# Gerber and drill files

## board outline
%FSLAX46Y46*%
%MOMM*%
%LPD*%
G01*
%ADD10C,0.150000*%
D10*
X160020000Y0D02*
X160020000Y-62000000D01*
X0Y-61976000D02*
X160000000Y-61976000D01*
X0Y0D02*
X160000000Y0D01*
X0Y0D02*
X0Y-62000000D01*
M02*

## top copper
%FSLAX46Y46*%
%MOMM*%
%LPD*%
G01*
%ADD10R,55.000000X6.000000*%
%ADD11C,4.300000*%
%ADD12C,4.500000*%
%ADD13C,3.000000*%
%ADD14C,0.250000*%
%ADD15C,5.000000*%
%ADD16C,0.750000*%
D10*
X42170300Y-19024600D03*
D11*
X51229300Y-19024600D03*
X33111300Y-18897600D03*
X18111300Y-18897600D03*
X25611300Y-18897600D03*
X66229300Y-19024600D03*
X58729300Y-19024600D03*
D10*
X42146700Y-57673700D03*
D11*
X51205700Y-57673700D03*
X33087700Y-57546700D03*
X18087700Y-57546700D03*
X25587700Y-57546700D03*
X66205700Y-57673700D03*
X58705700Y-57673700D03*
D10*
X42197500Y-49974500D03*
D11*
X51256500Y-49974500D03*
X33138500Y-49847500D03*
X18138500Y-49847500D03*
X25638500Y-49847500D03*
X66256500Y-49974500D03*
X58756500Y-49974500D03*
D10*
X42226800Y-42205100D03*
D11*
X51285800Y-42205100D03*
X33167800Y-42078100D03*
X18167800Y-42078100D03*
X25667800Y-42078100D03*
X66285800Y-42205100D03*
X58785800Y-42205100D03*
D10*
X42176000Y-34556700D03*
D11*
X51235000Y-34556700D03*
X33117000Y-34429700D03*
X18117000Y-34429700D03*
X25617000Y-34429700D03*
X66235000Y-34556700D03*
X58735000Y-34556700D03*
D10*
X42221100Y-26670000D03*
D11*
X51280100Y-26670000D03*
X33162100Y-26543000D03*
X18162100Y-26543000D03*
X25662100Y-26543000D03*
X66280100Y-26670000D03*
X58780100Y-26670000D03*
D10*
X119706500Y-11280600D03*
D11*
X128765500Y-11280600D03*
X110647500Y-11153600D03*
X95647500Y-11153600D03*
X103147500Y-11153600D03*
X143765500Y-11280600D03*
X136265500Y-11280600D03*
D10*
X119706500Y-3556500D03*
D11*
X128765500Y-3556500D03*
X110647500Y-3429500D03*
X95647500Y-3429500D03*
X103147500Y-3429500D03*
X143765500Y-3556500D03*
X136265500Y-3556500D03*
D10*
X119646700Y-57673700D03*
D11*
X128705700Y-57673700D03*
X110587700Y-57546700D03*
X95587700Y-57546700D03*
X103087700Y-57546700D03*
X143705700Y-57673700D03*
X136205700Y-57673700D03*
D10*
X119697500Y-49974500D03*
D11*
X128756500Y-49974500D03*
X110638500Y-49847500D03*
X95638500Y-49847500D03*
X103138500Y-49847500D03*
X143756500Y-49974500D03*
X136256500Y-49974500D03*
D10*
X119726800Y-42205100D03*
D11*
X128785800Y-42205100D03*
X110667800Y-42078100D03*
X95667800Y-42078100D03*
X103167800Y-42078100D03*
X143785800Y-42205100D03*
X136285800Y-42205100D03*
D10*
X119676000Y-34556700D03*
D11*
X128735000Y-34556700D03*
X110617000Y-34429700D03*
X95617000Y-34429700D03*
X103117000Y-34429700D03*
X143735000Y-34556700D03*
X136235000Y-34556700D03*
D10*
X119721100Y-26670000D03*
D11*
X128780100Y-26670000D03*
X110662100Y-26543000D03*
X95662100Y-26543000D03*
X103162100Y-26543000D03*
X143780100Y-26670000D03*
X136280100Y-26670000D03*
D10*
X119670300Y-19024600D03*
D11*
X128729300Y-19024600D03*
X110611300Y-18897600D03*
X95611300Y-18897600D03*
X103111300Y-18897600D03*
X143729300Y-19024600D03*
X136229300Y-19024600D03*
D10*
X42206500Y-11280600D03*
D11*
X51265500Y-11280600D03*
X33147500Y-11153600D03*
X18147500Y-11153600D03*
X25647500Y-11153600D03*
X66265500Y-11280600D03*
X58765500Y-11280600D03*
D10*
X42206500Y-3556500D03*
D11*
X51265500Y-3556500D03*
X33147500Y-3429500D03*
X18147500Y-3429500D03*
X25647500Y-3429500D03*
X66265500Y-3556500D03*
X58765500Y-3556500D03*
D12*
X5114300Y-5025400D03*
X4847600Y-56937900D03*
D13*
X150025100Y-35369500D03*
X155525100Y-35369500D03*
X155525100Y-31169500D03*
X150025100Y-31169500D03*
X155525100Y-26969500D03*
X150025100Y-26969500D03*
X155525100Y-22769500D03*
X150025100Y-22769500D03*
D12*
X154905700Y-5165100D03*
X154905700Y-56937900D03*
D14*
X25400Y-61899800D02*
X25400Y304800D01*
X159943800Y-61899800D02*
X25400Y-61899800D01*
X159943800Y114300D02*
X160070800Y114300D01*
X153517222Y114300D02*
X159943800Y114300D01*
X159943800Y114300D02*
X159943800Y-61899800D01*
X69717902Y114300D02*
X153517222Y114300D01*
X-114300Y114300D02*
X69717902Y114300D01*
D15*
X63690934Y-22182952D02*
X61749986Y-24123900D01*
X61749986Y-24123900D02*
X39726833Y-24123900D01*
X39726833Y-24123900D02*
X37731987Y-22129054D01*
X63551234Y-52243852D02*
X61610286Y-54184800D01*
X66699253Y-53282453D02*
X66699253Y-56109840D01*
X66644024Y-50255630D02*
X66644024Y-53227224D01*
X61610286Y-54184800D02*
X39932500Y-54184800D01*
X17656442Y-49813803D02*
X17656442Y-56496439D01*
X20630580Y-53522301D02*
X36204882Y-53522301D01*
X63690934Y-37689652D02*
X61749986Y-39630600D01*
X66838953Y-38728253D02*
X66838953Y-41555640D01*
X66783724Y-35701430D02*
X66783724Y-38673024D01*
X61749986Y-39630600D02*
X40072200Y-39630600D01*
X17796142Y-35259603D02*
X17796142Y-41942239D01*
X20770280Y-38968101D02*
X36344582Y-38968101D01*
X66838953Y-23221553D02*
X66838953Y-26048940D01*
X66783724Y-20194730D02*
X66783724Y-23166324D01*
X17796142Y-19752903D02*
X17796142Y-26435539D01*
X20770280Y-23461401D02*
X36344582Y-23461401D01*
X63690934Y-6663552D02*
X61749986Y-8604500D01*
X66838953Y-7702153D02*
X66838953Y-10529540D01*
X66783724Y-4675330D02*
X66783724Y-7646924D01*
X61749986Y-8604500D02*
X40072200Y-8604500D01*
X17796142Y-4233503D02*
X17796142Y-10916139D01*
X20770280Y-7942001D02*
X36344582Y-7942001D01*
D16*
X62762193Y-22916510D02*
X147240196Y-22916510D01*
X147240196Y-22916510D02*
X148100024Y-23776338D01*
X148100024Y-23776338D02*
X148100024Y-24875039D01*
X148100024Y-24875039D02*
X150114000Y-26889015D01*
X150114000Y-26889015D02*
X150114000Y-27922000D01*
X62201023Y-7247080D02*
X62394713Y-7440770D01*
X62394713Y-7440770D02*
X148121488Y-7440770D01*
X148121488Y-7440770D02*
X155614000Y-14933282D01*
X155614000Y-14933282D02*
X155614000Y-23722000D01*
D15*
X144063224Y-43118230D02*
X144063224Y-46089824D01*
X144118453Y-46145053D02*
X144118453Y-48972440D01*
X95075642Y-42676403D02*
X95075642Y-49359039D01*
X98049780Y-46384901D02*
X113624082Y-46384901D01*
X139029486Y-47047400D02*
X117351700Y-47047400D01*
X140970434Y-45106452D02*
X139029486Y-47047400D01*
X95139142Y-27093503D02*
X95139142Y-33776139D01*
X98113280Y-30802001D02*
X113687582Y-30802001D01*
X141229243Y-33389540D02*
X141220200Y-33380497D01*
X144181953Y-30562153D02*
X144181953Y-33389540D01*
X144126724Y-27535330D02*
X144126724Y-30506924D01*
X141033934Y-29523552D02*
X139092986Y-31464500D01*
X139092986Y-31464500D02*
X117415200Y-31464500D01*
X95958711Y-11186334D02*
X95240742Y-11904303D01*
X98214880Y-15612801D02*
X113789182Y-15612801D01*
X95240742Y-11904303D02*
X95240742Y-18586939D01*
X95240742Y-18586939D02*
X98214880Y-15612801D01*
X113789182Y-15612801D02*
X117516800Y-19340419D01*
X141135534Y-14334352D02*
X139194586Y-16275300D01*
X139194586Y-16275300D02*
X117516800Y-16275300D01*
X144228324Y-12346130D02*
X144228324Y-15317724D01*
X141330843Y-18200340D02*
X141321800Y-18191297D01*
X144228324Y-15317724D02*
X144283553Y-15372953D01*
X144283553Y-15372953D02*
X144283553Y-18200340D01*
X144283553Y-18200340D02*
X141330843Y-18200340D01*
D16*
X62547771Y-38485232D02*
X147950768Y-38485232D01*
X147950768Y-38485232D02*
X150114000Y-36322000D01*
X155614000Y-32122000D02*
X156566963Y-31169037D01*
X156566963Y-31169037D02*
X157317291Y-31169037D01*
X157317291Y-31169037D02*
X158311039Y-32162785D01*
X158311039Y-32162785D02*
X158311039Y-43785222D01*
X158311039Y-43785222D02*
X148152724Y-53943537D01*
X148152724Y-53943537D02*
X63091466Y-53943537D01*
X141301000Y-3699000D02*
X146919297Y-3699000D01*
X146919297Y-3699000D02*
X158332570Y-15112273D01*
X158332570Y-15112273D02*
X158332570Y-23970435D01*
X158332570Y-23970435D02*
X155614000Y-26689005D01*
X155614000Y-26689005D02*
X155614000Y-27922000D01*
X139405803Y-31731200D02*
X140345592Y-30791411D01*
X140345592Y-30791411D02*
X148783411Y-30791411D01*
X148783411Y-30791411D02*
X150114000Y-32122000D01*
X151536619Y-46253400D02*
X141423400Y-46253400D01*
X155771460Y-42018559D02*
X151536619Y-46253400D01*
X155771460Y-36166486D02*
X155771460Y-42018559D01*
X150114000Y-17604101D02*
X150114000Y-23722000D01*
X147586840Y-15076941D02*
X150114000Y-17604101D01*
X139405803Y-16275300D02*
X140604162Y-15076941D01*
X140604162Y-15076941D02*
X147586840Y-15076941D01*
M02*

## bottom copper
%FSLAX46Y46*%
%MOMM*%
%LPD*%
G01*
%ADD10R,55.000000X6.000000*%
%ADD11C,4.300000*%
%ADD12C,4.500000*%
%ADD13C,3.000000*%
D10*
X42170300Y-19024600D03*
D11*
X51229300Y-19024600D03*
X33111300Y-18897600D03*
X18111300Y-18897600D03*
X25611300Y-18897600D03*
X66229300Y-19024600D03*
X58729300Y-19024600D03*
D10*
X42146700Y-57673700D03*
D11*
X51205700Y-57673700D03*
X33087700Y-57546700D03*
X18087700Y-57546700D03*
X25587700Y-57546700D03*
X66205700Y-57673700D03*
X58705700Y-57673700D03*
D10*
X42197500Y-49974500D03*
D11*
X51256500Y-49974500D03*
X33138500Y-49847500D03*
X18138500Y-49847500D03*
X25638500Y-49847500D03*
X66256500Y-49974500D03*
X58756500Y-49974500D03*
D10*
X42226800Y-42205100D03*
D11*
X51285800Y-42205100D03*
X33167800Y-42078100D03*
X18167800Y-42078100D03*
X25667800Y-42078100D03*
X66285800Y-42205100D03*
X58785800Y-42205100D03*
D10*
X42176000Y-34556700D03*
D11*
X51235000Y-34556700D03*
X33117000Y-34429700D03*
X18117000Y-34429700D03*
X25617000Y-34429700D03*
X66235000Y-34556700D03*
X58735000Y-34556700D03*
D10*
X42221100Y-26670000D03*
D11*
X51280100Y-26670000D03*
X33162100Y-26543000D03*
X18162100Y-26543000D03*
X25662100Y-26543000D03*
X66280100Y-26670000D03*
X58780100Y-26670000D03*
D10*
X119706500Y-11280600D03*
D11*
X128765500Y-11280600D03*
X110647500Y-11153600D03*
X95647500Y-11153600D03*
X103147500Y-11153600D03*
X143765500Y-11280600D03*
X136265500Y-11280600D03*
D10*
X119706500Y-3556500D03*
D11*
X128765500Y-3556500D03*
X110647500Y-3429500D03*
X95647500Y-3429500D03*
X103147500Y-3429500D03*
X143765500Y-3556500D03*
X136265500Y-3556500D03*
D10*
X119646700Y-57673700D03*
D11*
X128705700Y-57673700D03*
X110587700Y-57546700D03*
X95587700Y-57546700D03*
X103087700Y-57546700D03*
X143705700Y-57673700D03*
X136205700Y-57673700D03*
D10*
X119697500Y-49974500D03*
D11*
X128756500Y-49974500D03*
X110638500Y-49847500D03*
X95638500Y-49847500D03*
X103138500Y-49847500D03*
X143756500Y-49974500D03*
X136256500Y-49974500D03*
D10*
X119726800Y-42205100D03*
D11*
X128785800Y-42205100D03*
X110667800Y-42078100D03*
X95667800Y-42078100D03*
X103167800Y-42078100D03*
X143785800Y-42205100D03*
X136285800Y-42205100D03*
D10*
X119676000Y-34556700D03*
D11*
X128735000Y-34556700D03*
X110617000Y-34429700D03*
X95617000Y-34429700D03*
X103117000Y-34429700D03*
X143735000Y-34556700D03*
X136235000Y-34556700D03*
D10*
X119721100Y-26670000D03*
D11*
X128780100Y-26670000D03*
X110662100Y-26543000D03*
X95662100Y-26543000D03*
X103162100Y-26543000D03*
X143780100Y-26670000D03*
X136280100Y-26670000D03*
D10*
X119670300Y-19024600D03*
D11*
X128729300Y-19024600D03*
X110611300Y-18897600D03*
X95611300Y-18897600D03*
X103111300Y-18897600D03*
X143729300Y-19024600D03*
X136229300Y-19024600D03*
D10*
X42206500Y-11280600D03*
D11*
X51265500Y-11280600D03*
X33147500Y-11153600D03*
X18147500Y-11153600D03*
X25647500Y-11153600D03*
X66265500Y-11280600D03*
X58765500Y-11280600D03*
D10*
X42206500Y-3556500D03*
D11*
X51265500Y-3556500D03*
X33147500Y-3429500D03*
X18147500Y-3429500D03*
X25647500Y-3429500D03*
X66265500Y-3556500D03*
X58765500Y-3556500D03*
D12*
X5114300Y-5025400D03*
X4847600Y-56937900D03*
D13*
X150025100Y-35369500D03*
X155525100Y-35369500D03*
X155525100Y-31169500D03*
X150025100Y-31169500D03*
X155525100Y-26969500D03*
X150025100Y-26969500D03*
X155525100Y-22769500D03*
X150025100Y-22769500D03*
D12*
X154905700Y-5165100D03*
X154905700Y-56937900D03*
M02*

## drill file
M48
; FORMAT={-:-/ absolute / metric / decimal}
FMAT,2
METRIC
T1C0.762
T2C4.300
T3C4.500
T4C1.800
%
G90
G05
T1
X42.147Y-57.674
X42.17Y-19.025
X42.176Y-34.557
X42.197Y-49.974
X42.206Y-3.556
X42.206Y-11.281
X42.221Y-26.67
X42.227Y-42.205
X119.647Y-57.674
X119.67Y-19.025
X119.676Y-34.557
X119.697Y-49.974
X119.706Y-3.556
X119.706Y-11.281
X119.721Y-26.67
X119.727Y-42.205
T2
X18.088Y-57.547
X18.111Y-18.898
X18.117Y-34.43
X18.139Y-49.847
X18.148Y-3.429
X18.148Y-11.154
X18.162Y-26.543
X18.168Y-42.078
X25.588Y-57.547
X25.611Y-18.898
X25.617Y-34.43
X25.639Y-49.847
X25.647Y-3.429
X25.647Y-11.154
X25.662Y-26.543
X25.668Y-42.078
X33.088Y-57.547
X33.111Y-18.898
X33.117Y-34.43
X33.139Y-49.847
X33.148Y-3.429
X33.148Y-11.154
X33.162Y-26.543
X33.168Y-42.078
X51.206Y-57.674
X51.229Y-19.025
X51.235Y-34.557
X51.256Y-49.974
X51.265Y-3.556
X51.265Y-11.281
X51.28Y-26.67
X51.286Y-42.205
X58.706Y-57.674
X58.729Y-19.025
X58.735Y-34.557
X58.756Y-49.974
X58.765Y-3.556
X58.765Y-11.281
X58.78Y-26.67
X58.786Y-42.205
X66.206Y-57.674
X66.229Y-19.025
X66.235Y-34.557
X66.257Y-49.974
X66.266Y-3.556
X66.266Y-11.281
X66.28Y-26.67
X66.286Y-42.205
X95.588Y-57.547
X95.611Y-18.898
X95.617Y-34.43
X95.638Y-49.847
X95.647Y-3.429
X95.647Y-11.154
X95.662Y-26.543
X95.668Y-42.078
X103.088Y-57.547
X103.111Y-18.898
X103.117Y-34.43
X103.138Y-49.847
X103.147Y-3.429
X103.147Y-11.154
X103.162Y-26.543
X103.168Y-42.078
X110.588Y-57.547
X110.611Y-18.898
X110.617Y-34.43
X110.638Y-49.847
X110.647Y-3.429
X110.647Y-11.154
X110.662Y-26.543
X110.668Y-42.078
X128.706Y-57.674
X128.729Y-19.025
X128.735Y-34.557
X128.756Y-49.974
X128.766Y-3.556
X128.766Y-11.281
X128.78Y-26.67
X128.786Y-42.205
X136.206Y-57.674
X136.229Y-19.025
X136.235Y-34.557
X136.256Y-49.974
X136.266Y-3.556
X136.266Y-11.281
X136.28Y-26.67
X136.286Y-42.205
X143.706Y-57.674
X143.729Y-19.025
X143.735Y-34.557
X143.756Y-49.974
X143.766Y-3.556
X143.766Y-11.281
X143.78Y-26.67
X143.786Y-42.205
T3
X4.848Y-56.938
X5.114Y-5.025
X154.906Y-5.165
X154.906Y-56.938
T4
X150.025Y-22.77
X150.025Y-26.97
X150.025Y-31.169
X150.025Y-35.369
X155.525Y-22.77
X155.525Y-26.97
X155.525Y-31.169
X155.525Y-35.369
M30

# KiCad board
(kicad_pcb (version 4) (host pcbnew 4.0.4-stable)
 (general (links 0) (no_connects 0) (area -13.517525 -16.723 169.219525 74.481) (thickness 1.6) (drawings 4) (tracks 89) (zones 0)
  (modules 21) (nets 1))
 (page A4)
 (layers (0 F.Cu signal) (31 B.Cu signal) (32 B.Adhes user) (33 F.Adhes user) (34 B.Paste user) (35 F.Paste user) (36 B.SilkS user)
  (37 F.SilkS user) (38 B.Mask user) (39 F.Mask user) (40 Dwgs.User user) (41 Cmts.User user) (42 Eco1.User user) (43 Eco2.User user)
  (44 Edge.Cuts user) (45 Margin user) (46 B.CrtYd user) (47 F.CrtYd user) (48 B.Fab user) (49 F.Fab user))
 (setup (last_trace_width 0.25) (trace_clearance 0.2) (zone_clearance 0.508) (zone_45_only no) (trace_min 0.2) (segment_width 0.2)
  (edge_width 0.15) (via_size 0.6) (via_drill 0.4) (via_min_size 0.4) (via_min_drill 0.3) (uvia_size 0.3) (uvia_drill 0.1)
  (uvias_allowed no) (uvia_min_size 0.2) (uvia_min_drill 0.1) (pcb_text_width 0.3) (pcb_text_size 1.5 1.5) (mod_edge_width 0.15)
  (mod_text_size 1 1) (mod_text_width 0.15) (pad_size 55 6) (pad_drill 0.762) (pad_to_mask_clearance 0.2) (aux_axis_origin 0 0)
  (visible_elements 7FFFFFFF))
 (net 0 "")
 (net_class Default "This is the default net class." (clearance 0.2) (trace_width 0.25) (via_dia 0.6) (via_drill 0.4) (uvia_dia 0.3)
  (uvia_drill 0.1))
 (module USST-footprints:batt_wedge (layer F.Cu) (at 42.1703 19.0246)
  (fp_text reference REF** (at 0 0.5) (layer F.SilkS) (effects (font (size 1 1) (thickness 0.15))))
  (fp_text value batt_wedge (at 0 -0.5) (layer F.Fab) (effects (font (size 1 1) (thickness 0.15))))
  (pad 1 thru_hole rect (at 0 0) (size 55 6) (drill 0.762) (layers F.Cu F.Paste))
  (pad "" thru_hole circle (at 9.059 0) (size 4.3 4.3) (drill 4.3) (layers *.Cu *.Mask))
  (pad "" thru_hole circle (at -9.059 -0.127) (size 4.3 4.3) (drill 4.3) (layers *.Cu *.Mask))
  (pad "" thru_hole circle (at -24.059 -0.127) (size 4.3 4.3) (drill 4.3) (layers *.Cu *.Mask))
  (pad "" thru_hole circle (at -16.559 -0.127) (size 4.3 4.3) (drill 4.3) (layers *.Cu *.Mask))
  (pad "" thru_hole circle (at 24.059 0) (size 4.3 4.3) (drill 4.3) (layers *.Cu *.Mask))
  (pad "" thru_hole circle (at 16.559 0) (size 4.3 4.3) (drill 4.3) (layers *.Cu *.Mask)))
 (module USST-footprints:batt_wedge (layer F.Cu) (at 42.1467 57.6737)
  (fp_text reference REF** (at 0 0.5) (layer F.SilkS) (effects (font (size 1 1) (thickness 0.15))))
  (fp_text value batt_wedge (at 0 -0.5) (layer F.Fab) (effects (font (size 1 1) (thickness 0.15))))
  (pad 1 thru_hole rect (at 0 0) (size 55 6) (drill 0.762) (layers F.Cu F.Paste))
  (pad "" thru_hole circle (at 9.059 0) (size 4.3 4.3) (drill 4.3) (layers *.Cu *.Mask))
  (pad "" thru_hole circle (at -9.059 -0.127) (size 4.3 4.3) (drill 4.3) (layers *.Cu *.Mask))
  (pad "" thru_hole circle (at -24.059 -0.127) (size 4.3 4.3) (drill 4.3) (layers *.Cu *.Mask))
  (pad "" thru_hole circle (at -16.559 -0.127) (size 4.3 4.3) (drill 4.3) (layers *.Cu *.Mask))
  (pad "" thru_hole circle (at 24.059 0) (size 4.3 4.3) (drill 4.3) (layers *.Cu *.Mask))
  (pad "" thru_hole circle (at 16.559 0) (size 4.3 4.3) (drill 4.3) (layers *.Cu *.Mask)))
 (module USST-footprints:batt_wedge (layer F.Cu) (at 42.1975 49.9745)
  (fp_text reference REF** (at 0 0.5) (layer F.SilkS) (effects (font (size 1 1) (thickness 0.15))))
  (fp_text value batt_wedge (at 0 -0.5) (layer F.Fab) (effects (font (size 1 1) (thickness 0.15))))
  (pad 1 thru_hole rect (at 0 0) (size 55 6) (drill 0.762) (layers F.Cu F.Paste))
  (pad "" thru_hole circle (at 9.059 0) (size 4.3 4.3) (drill 4.3) (layers *.Cu *.Mask))
  (pad "" thru_hole circle (at -9.059 -0.127) (size 4.3 4.3) (drill 4.3) (layers *.Cu *.Mask))
  (pad "" thru_hole circle (at -24.059 -0.127) (size 4.3 4.3) (drill 4.3) (layers *.Cu *.Mask))
  (pad "" thru_hole circle (at -16.559 -0.127) (size 4.3 4.3) (drill 4.3) (layers *.Cu *.Mask))
  (pad "" thru_hole circle (at 24.059 0) (size 4.3 4.3) (drill 4.3) (layers *.Cu *.Mask))
  (pad "" thru_hole circle (at 16.559 0) (size 4.3 4.3) (drill 4.3) (layers *.Cu *.Mask)))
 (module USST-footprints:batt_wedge (layer F.Cu) (at 42.2268 42.2051)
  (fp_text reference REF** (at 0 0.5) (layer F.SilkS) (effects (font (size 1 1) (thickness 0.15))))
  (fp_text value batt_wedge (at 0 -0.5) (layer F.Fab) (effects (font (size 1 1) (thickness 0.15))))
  (pad 1 thru_hole rect (at 0 0) (size 55 6) (drill 0.762) (layers F.Cu F.Paste))
  (pad "" thru_hole circle (at 9.059 0) (size 4.3 4.3) (drill 4.3) (layers *.Cu *.Mask))
  (pad "" thru_hole circle (at -9.059 -0.127) (size 4.3 4.3) (drill 4.3) (layers *.Cu *.Mask))
  (pad "" thru_hole circle (at -24.059 -0.127) (size 4.3 4.3) (drill 4.3) (layers *.Cu *.Mask))
  (pad "" thru_hole circle (at -16.559 -0.127) (size 4.3 4.3) (drill 4.3) (layers *.Cu *.Mask))
  (pad "" thru_hole circle (at 24.059 0) (size 4.3 4.3) (drill 4.3) (layers *.Cu *.Mask))
  (pad "" thru_hole circle (at 16.559 0) (size 4.3 4.3) (drill 4.3) (layers *.Cu *.Mask)))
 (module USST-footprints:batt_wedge (layer F.Cu) (at 42.176 34.5567)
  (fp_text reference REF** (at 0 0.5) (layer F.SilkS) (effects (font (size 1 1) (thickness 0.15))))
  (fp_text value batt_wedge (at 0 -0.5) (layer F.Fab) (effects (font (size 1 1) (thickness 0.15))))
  (pad 1 thru_hole rect (at 0 0) (size 55 6) (drill 0.762) (layers F.Cu F.Paste))
  (pad "" thru_hole circle (at 9.059 0) (size 4.3 4.3) (drill 4.3) (layers *.Cu *.Mask))
  (pad "" thru_hole circle (at -9.059 -0.127) (size 4.3 4.3) (drill 4.3) (layers *.Cu *.Mask))
  (pad "" thru_hole circle (at -24.059 -0.127) (size 4.3 4.3) (drill 4.3) (layers *.Cu *.Mask))
  (pad "" thru_hole circle (at -16.559 -0.127) (size 4.3 4.3) (drill 4.3) (layers *.Cu *.Mask))
  (pad "" thru_hole circle (at 24.059 0) (size 4.3 4.3) (drill 4.3) (layers *.Cu *.Mask))
  (pad "" thru_hole circle (at 16.559 0) (size 4.3 4.3) (drill 4.3) (layers *.Cu *.Mask)))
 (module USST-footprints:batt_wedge (layer F.Cu) (at 42.2211 26.67)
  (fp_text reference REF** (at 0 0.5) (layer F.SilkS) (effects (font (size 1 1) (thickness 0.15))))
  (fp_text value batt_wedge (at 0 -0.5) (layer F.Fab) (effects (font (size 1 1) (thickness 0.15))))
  (pad 1 thru_hole rect (at 0 0) (size 55 6) (drill 0.762) (layers F.Cu F.Paste))
  (pad "" thru_hole circle (at 9.059 0) (size 4.3 4.3) (drill 4.3) (layers *.Cu *.Mask))
  (pad "" thru_hole circle (at -9.059 -0.127) (size 4.3 4.3) (drill 4.3) (layers *.Cu *.Mask))
  (pad "" thru_hole circle (at -24.059 -0.127) (size 4.3 4.3) (drill 4.3) (layers *.Cu *.Mask))
  (pad "" thru_hole circle (at -16.559 -0.127) (size 4.3 4.3) (drill 4.3) (layers *.Cu *.Mask))
  (pad "" thru_hole circle (at 24.059 0) (size 4.3 4.3) (drill 4.3) (layers *.Cu *.Mask))
  (pad "" thru_hole circle (at 16.559 0) (size 4.3 4.3) (drill 4.3) (layers *.Cu *.Mask)))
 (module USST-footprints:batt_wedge (layer F.Cu) (at 119.7065 11.2806)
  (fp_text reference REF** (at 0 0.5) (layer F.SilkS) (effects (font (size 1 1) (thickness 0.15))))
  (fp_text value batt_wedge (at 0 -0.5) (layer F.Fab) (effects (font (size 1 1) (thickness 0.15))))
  (pad 1 thru_hole rect (at 0 0) (size 55 6) (drill 0.762) (layers F.Cu F.Paste))
  (pad "" thru_hole circle (at 9.059 0) (size 4.3 4.3) (drill 4.3) (layers *.Cu *.Mask))
  (pad "" thru_hole circle (at -9.059 -0.127) (size 4.3 4.3) (drill 4.3) (layers *.Cu *.Mask))
  (pad "" thru_hole circle (at -24.059 -0.127) (size 4.3 4.3) (drill 4.3) (layers *.Cu *.Mask))
  (pad "" thru_hole circle (at -16.559 -0.127) (size 4.3 4.3) (drill 4.3) (layers *.Cu *.Mask))
  (pad "" thru_hole circle (at 24.059 0) (size 4.3 4.3) (drill 4.3) (layers *.Cu *.Mask))
  (pad "" thru_hole circle (at 16.559 0) (size 4.3 4.3) (drill 4.3) (layers *.Cu *.Mask)))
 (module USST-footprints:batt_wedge (layer F.Cu) (at 119.7065 3.5565)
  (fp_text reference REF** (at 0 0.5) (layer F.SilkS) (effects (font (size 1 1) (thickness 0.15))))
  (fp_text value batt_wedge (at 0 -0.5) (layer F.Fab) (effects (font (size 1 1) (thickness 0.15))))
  (pad 1 thru_hole rect (at 0 0) (size 55 6) (drill 0.762) (layers F.Cu F.Paste))
  (pad "" thru_hole circle (at 9.059 0) (size 4.3 4.3) (drill 4.3) (layers *.Cu *.Mask))
  (pad "" thru_hole circle (at -9.059 -0.127) (size 4.3 4.3) (drill 4.3) (layers *.Cu *.Mask))
  (pad "" thru_hole circle (at -24.059 -0.127) (size 4.3 4.3) (drill 4.3) (layers *.Cu *.Mask))
  (pad "" thru_hole circle (at -16.559 -0.127) (size 4.3 4.3) (drill 4.3) (layers *.Cu *.Mask))
  (pad "" thru_hole circle (at 24.059 0) (size 4.3 4.3) (drill 4.3) (layers *.Cu *.Mask))
  (pad "" thru_hole circle (at 16.559 0) (size 4.3 4.3) (drill 4.3) (layers *.Cu *.Mask)))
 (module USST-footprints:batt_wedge (layer F.Cu) (at 119.6467 57.6737)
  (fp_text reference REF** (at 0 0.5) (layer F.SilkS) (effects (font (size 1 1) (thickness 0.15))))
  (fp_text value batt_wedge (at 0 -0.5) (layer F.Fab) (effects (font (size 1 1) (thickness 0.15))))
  (pad 1 thru_hole rect (at 0 0) (size 55 6) (drill 0.762) (layers F.Cu F.Paste))
  (pad "" thru_hole circle (at 9.059 0) (size 4.3 4.3) (drill 4.3) (layers *.Cu *.Mask))
  (pad "" thru_hole circle (at -9.059 -0.127) (size 4.3 4.3) (drill 4.3) (layers *.Cu *.Mask))
  (pad "" thru_hole circle (at -24.059 -0.127) (size 4.3 4.3) (drill 4.3) (layers *.Cu *.Mask))
  (pad "" thru_hole circle (at -16.559 -0.127) (size 4.3 4.3) (drill 4.3) (layers *.Cu *.Mask))
  (pad "" thru_hole circle (at 24.059 0) (size 4.3 4.3) (drill 4.3) (layers *.Cu *.Mask))
  (pad "" thru_hole circle (at 16.559 0) (size 4.3 4.3) (drill 4.3) (layers *.Cu *.Mask)))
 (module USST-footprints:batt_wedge (layer F.Cu) (at 119.6975 49.9745)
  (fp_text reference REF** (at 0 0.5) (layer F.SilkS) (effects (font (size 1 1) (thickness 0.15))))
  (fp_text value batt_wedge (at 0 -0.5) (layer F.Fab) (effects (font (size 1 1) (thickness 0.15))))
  (pad 1 thru_hole rect (at 0 0) (size 55 6) (drill 0.762) (layers F.Cu F.Paste))
  (pad "" thru_hole circle (at 9.059 0) (size 4.3 4.3) (drill 4.3) (layers *.Cu *.Mask))
  (pad "" thru_hole circle (at -9.059 -0.127) (size 4.3 4.3) (drill 4.3) (layers *.Cu *.Mask))
  (pad "" thru_hole circle (at -24.059 -0.127) (size 4.3 4.3) (drill 4.3) (layers *.Cu *.Mask))
  (pad "" thru_hole circle (at -16.559 -0.127) (size 4.3 4.3) (drill 4.3) (layers *.Cu *.Mask))
  (pad "" thru_hole circle (at 24.059 0) (size 4.3 4.3) (drill 4.3) (layers *.Cu *.Mask))
  (pad "" thru_hole circle (at 16.559 0) (size 4.3 4.3) (drill 4.3) (layers *.Cu *.Mask)))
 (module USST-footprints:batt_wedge (layer F.Cu) (at 119.7268 42.2051)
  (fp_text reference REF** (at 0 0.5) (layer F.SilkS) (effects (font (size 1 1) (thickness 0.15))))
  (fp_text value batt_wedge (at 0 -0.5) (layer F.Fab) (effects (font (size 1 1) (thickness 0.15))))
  (pad 1 thru_hole rect (at 0 0) (size 55 6) (drill 0.762) (layers F.Cu F.Paste))
  (pad "" thru_hole circle (at 9.059 0) (size 4.3 4.3) (drill 4.3) (layers *.Cu *.Mask))
  (pad "" thru_hole circle (at -9.059 -0.127) (size 4.3 4.3) (drill 4.3) (layers *.Cu *.Mask))
  (pad "" thru_hole circle (at -24.059 -0.127) (size 4.3 4.3) (drill 4.3) (layers *.Cu *.Mask))
  (pad "" thru_hole circle (at -16.559 -0.127) (size 4.3 4.3) (drill 4.3) (layers *.Cu *.Mask))
  (pad "" thru_hole circle (at 24.059 0) (size 4.3 4.3) (drill 4.3) (layers *.Cu *.Mask))
  (pad "" thru_hole circle (at 16.559 0) (size 4.3 4.3) (drill 4.3) (layers *.Cu *.Mask)))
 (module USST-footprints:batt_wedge (layer F.Cu) (at 119.676 34.5567)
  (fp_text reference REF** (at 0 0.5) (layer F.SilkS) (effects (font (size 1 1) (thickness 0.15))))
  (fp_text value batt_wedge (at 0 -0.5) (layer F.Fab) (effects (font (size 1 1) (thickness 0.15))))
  (pad 1 thru_hole rect (at 0 0) (size 55 6) (drill 0.762) (layers F.Cu F.Paste))
  (pad "" thru_hole circle (at 9.059 0) (size 4.3 4.3) (drill 4.3) (layers *.Cu *.Mask))
  (pad "" thru_hole circle (at -9.059 -0.127) (size 4.3 4.3) (drill 4.3) (layers *.Cu *.Mask))
  (pad "" thru_hole circle (at -24.059 -0.127) (size 4.3 4.3) (drill 4.3) (layers *.Cu *.Mask))
  (pad "" thru_hole circle (at -16.559 -0.127) (size 4.3 4.3) (drill 4.3) (layers *.Cu *.Mask))
  (pad "" thru_hole circle (at 24.059 0) (size 4.3 4.3) (drill 4.3) (layers *.Cu *.Mask))
  (pad "" thru_hole circle (at 16.559 0) (size 4.3 4.3) (drill 4.3) (layers *.Cu *.Mask)))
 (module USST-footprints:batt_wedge (layer F.Cu) (at 119.7211 26.67)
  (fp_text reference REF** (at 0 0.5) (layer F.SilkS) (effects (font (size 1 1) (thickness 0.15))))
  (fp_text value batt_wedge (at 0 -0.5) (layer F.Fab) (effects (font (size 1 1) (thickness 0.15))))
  (pad 1 thru_hole rect (at 0 0) (size 55 6) (drill 0.762) (layers F.Cu F.Paste))
  (pad "" thru_hole circle (at 9.059 0) (size 4.3 4.3) (drill 4.3) (layers *.Cu *.Mask))
  (pad "" thru_hole circle (at -9.059 -0.127) (size 4.3 4.3) (drill 4.3) (layers *.Cu *.Mask))
  (pad "" thru_hole circle (at -24.059 -0.127) (size 4.3 4.3) (drill 4.3) (layers *.Cu *.Mask))
  (pad "" thru_hole circle (at -16.559 -0.127) (size 4.3 4.3) (drill 4.3) (layers *.Cu *.Mask))
  (pad "" thru_hole circle (at 24.059 0) (size 4.3 4.3) (drill 4.3) (layers *.Cu *.Mask))
  (pad "" thru_hole circle (at 16.559 0) (size 4.3 4.3) (drill 4.3) (layers *.Cu *.Mask)))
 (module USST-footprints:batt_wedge (layer F.Cu) (at 119.6703 19.0246)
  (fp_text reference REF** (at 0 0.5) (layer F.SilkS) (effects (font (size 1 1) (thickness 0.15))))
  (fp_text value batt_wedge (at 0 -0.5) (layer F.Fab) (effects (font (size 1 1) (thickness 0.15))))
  (pad 1 thru_hole rect (at 0 0) (size 55 6) (drill 0.762) (layers F.Cu F.Paste))
  (pad "" thru_hole circle (at 9.059 0) (size 4.3 4.3) (drill 4.3) (layers *.Cu *.Mask))
  (pad "" thru_hole circle (at -9.059 -0.127) (size 4.3 4.3) (drill 4.3) (layers *.Cu *.Mask))
  (pad "" thru_hole circle (at -24.059 -0.127) (size 4.3 4.3) (drill 4.3) (layers *.Cu *.Mask))
  (pad "" thru_hole circle (at -16.559 -0.127) (size 4.3 4.3) (drill 4.3) (layers *.Cu *.Mask))
  (pad "" thru_hole circle (at 24.059 0) (size 4.3 4.3) (drill 4.3) (layers *.Cu *.Mask))
  (pad "" thru_hole circle (at 16.559 0) (size 4.3 4.3) (drill 4.3) (layers *.Cu *.Mask)))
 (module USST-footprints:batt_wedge (layer F.Cu) (at 42.2065 11.2806)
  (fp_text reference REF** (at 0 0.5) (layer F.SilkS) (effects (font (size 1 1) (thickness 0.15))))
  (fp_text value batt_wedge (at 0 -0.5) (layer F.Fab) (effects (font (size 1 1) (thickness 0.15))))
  (pad 1 thru_hole rect (at 0 0) (size 55 6) (drill 0.762) (layers F.Cu F.Paste))
  (pad "" thru_hole circle (at 9.059 0) (size 4.3 4.3) (drill 4.3) (layers *.Cu *.Mask))
  (pad "" thru_hole circle (at -9.059 -0.127) (size 4.3 4.3) (drill 4.3) (layers *.Cu *.Mask))
  (pad "" thru_hole circle (at -24.059 -0.127) (size 4.3 4.3) (drill 4.3) (layers *.Cu *.Mask))
  (pad "" thru_hole circle (at -16.559 -0.127) (size 4.3 4.3) (drill 4.3) (layers *.Cu *.Mask))
  (pad "" thru_hole circle (at 24.059 0) (size 4.3 4.3) (drill 4.3) (layers *.Cu *.Mask))
  (pad "" thru_hole circle (at 16.559 0) (size 4.3 4.3) (drill 4.3) (layers *.Cu *.Mask)))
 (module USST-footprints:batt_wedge (layer F.Cu) (at 42.2065 3.5565)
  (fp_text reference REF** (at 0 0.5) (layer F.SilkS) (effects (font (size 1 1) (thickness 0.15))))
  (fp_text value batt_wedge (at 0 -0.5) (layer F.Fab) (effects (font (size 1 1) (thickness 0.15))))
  (pad 1 thru_hole rect (at 0 0) (size 55 6) (drill 0.762) (layers F.Cu F.Paste))
  (pad "" thru_hole circle (at 9.059 0) (size 4.3 4.3) (drill 4.3) (layers *.Cu *.Mask))
  (pad "" thru_hole circle (at -9.059 -0.127) (size 4.3 4.3) (drill 4.3) (layers *.Cu *.Mask))
  (pad "" thru_hole circle (at -24.059 -0.127) (size 4.3 4.3) (drill 4.3) (layers *.Cu *.Mask))
  (pad "" thru_hole circle (at -16.559 -0.127) (size 4.3 4.3) (drill 4.3) (layers *.Cu *.Mask))
  (pad "" thru_hole circle (at 24.059 0) (size 4.3 4.3) (drill 4.3) (layers *.Cu *.Mask))
  (pad "" thru_hole circle (at 16.559 0) (size 4.3 4.3) (drill 4.3) (layers *.Cu *.Mask)))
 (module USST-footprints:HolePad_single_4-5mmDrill (layer F.Cu) (at 5.1143 5.0254)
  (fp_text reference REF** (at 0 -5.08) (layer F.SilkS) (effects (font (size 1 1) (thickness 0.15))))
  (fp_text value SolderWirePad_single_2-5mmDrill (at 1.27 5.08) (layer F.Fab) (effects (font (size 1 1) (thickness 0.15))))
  (pad "" thru_hole circle (at 0 0) (size 4.5 4.5) (drill 4.5) (layers *.Cu *.Mask)))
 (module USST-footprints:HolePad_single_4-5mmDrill (layer F.Cu) (at 4.8476 56.9379)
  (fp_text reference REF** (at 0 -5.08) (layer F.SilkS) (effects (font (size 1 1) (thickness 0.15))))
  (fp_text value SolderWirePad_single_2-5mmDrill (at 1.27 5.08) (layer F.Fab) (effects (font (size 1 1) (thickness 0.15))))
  (pad "" thru_hole circle (at 0 0) (size 4.5 4.5) (drill 4.5) (layers *.Cu *.Mask)))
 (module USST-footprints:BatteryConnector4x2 (layer F.Cu) (at 150.0251 35.3695)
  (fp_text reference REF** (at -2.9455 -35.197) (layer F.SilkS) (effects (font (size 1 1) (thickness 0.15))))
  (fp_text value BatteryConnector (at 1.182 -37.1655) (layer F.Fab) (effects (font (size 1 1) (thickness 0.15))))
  (pad "" np_thru_hole circle (at 0 0) (size 3 3) (drill 1.8) (layers *.Cu))
  (pad "" np_thru_hole circle (at 5.5 0) (size 3 3) (drill 1.8) (layers *.Cu))
  (pad "" np_thru_hole circle (at 5.5 -4.2) (size 3 3) (drill 1.8) (layers *.Cu))
  (pad "" np_thru_hole circle (at 0 -4.2) (size 3 3) (drill 1.8) (layers *.Cu))
  (pad "" np_thru_hole circle (at 5.5 -8.4) (size 3 3) (drill 1.8) (layers *.Cu))
  (pad "" np_thru_hole circle (at 0 -8.4) (size 3 3) (drill 1.8) (layers *.Cu))
  (pad "" np_thru_hole circle (at 5.5 -12.6) (size 3 3) (drill 1.8) (layers *.Cu))
  (pad "" np_thru_hole circle (at 0 -12.6) (size 3 3) (drill 1.8) (layers *.Cu)))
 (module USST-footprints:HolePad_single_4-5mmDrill (layer F.Cu) (at 154.9057 5.1651)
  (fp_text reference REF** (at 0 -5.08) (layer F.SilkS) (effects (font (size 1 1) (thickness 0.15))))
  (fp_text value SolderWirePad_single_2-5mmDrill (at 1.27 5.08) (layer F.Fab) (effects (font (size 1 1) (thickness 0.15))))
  (pad "" thru_hole circle (at 0 0) (size 4.5 4.5) (drill 4.5) (layers *.Cu *.Mask)))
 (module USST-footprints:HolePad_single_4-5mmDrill (layer F.Cu) (at 154.9057 56.9379)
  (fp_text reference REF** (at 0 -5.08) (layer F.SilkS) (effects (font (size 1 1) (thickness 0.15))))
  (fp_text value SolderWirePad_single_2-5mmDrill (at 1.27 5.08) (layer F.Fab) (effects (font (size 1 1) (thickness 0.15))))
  (pad "" thru_hole circle (at 0 0) (size 4.5 4.5) (drill 4.5) (layers *.Cu *.Mask)))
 (gr_line (start 160.02 0) (end 160.02 62) (layer Edge.Cuts) (width 0.15))
 (gr_line (start 0 61.976) (end 160 61.976) (layer Edge.Cuts) (width 0.15))
 (gr_line (start 0 0) (end 160 0) (layer Edge.Cuts) (width 0.15))
 (gr_line (start 0 0) (end 0 62) (layer Edge.Cuts) (width 0.15))
 (segment (start 0.0254 61.8998) (end 0.0254 -0.3048) (width 0.25) (layer F.Cu) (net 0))
 (segment (start 159.9438 61.8998) (end 0.0254 61.8998) (width 0.25) (layer F.Cu) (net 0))
 (segment (start 159.9438 -0.1143) (end 160.0708 -0.1143) (width 0.25) (layer F.Cu) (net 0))
 (segment (start 153.517222 -0.1143) (end 159.9438 -0.1143) (width 0.25) (layer F.Cu) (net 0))
 (segment (start 159.9438 -0.1143) (end 159.9438 61.8998) (width 0.25) (layer F.Cu) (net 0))
 (segment (start 69.717902 -0.1143) (end 153.517222 -0.1143) (width 0.25) (layer F.Cu) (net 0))
 (segment (start -0.1143 -0.1143) (end 69.717902 -0.1143) (width 0.25) (layer F.Cu) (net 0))
 (segment (start 63.690934 22.182952) (end 61.749986 24.1239) (width 5) (layer F.Cu) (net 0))
 (segment (start 61.749986 24.1239) (end 39.726833 24.1239) (width 5) (layer F.Cu) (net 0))
 (segment (start 39.726833 24.1239) (end 37.731987 22.129054) (width 5) (layer F.Cu) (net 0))
 (segment (start 63.551234 52.243852) (end 61.610286 54.1848) (width 5) (layer F.Cu) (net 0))
 (segment (start 66.699253 53.282453) (end 66.699253 56.10984) (width 5) (layer F.Cu) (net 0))
 (segment (start 66.644024 50.25563) (end 66.644024 53.227224) (width 5) (layer F.Cu) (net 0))
 (segment (start 61.610286 54.1848) (end 39.9325 54.1848) (width 5) (layer F.Cu) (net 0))
 (segment (start 17.656442 49.813803) (end 17.656442 56.496439) (width 5) (layer F.Cu) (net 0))
 (segment (start 20.63058 53.522301) (end 36.204882 53.522301) (width 5) (layer F.Cu) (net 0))
 (segment (start 63.690934 37.689652) (end 61.749986 39.6306) (width 5) (layer F.Cu) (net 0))
 (segment (start 66.838953 38.728253) (end 66.838953 41.55564) (width 5) (layer F.Cu) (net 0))
 (segment (start 66.783724 35.70143) (end 66.783724 38.673024) (width 5) (layer F.Cu) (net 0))
 (segment (start 61.749986 39.6306) (end 40.0722 39.6306) (width 5) (layer F.Cu) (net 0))
 (segment (start 17.796142 35.259603) (end 17.796142 41.942239) (width 5) (layer F.Cu) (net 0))
 (segment (start 20.77028 38.968101) (end 36.344582 38.968101) (width 5) (layer F.Cu) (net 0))
 (segment (start 66.838953 23.221553) (end 66.838953 26.04894) (width 5) (layer F.Cu) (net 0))
 (segment (start 66.783724 20.19473) (end 66.783724 23.166324) (width 5) (layer F.Cu) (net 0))
 (segment (start 17.796142 19.752903) (end 17.796142 26.435539) (width 5) (layer F.Cu) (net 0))
 (segment (start 20.77028 23.461401) (end 36.344582 23.461401) (width 5) (layer F.Cu) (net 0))
 (segment (start 63.690934 6.663552) (end 61.749986 8.6045) (width 5) (layer F.Cu) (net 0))
 (segment (start 66.838953 7.702153) (end 66.838953 10.52954) (width 5) (layer F.Cu) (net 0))
 (segment (start 66.783724 4.67533) (end 66.783724 7.646924) (width 5) (layer F.Cu) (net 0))
 (segment (start 61.749986 8.6045) (end 40.0722 8.6045) (width 5) (layer F.Cu) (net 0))
 (segment (start 17.796142 4.233503) (end 17.796142 10.916139) (width 5) (layer F.Cu) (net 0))
 (segment (start 20.77028 7.942001) (end 36.344582 7.942001) (width 5) (layer F.Cu) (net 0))
 (segment (start 62.762193 22.91651) (end 147.240196 22.91651) (width 0.75) (layer F.Cu) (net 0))
 (segment (start 147.240196 22.91651) (end 148.100024 23.776338) (width 0.75) (layer F.Cu) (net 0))
 (segment (start 148.100024 23.776338) (end 148.100024 24.875039) (width 0.75) (layer F.Cu) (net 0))
 (segment (start 148.100024 24.875039) (end 150.114 26.889015) (width 0.75) (layer F.Cu) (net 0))
 (segment (start 150.114 26.889015) (end 150.114 27.922) (width 0.75) (layer F.Cu) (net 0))
 (segment (start 62.201023 7.24708) (end 62.394713 7.44077) (width 0.75) (layer F.Cu) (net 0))
 (segment (start 62.394713 7.44077) (end 148.121488 7.44077) (width 0.75) (layer F.Cu) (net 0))
 (segment (start 148.121488 7.44077) (end 155.614 14.933282) (width 0.75) (layer F.Cu) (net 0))
 (segment (start 155.614 14.933282) (end 155.614 23.722) (width 0.75) (layer F.Cu) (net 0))
 (segment (start 144.063224 43.11823) (end 144.063224 46.089824) (width 5) (layer F.Cu) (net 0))
 (segment (start 144.118453 46.145053) (end 144.118453 48.97244) (width 5) (layer F.Cu) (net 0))
 (segment (start 95.075642 42.676403) (end 95.075642 49.359039) (width 5) (layer F.Cu) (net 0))
 (segment (start 98.04978 46.384901) (end 113.624082 46.384901) (width 5) (layer F.Cu) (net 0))
 (segment (start 139.029486 47.0474) (end 117.3517 47.0474) (width 5) (layer F.Cu) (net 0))
 (segment (start 140.970434 45.106452) (end 139.029486 47.0474) (width 5) (layer F.Cu) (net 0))
 (segment (start 95.139142 27.093503) (end 95.139142 33.776139) (width 5) (layer F.Cu) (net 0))
 (segment (start 98.11328 30.802001) (end 113.687582 30.802001) (width 5) (layer F.Cu) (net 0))
 (segment (start 141.229243 33.38954) (end 141.2202 33.380497) (width 5) (layer F.Cu) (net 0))
 (segment (start 144.181953 30.562153) (end 144.181953 33.38954) (width 5) (layer F.Cu) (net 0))
 (segment (start 144.126724 27.53533) (end 144.126724 30.506924) (width 5) (layer F.Cu) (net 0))
 (segment (start 141.033934 29.523552) (end 139.092986 31.4645) (width 5) (layer F.Cu) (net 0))
 (segment (start 139.092986 31.4645) (end 117.4152 31.4645) (width 5) (layer F.Cu) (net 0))
 (segment (start 95.958711 11.186334) (end 95.240742 11.904303) (width 5) (layer F.Cu) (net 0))
 (segment (start 98.21488 15.612801) (end 113.789182 15.612801) (width 5) (layer F.Cu) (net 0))
 (segment (start 95.240742 11.904303) (end 95.240742 18.586939) (width 5) (layer F.Cu) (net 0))
 (segment (start 95.240742 18.586939) (end 98.21488 15.612801) (width 5) (layer F.Cu) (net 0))
 (segment (start 113.789182 15.612801) (end 117.5168 19.340419) (width 5) (layer F.Cu) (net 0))
 (segment (start 141.135534 14.334352) (end 139.194586 16.2753) (width 5) (layer F.Cu) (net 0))
 (segment (start 139.194586 16.2753) (end 117.5168 16.2753) (width 5) (layer F.Cu) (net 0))
 (segment (start 144.228324 12.34613) (end 144.228324 15.317724) (width 5) (layer F.Cu) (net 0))
 (segment (start 141.330843 18.20034) (end 141.3218 18.191297) (width 5) (layer F.Cu) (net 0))
 (segment (start 144.228324 15.317724) (end 144.283553 15.372953) (width 5) (layer F.Cu) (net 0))
 (segment (start 144.283553 15.372953) (end 144.283553 18.20034) (width 5) (layer F.Cu) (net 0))
 (segment (start 144.283553 18.20034) (end 141.330843 18.20034) (width 5) (layer F.Cu) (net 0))
 (segment (start 62.547771 38.485232) (end 147.950768 38.485232) (width 0.75) (layer F.Cu) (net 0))
 (segment (start 147.950768 38.485232) (end 150.114 36.322) (width 0.75) (layer F.Cu) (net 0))
 (segment (start 155.614 32.122) (end 156.566963 31.169037) (width 0.75) (layer F.Cu) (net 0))
 (segment (start 156.566963 31.169037) (end 157.317291 31.169037) (width 0.75) (layer F.Cu) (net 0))
 (segment (start 157.317291 31.169037) (end 158.311039 32.162785) (width 0.75) (layer F.Cu) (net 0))
 (segment (start 158.311039 32.162785) (end 158.311039 43.785222) (width 0.75) (layer F.Cu) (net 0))
 (segment (start 158.311039 43.785222) (end 148.152724 53.943537) (width 0.75) (layer F.Cu) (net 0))
 (segment (start 148.152724 53.943537) (end 63.091466 53.943537) (width 0.75) (layer F.Cu) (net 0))
 (segment (start 141.301 3.699) (end 146.919297 3.699) (width 0.75) (layer F.Cu) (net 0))
 (segment (start 146.919297 3.699) (end 158.33257 15.112273) (width 0.75) (layer F.Cu) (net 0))
 (segment (start 158.33257 15.112273) (end 158.33257 23.970435) (width 0.75) (layer F.Cu) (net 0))
 (segment (start 158.33257 23.970435) (end 155.614 26.689005) (width 0.75) (layer F.Cu) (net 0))
 (segment (start 155.614 26.689005) (end 155.614 27.922) (width 0.75) (layer F.Cu) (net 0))
 (segment (start 139.405803 31.7312) (end 140.345592 30.791411) (width 0.75) (layer F.Cu) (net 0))
 (segment (start 140.345592 30.791411) (end 148.783411 30.791411) (width 0.75) (layer F.Cu) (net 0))
 (segment (start 148.783411 30.791411) (end 150.114 32.122) (width 0.75) (layer F.Cu) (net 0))
 (segment (start 151.536619 46.2534) (end 141.4234 46.2534) (width 0.75) (layer F.Cu) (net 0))
 (segment (start 155.77146 42.018559) (end 151.536619 46.2534) (width 0.75) (layer F.Cu) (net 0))
 (segment (start 155.77146 36.166486) (end 155.77146 42.018559) (width 0.75) (layer F.Cu) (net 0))
 (segment (start 150.114 17.604101) (end 150.114 23.722) (width 0.75) (layer F.Cu) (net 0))
 (segment (start 147.58684 15.076941) (end 150.114 17.604101) (width 0.75) (layer F.Cu) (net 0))
 (segment (start 139.405803 16.2753) (end 140.604162 15.076941) (width 0.75) (layer F.Cu) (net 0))
 (segment (start 140.604162 15.076941) (end 147.58684 15.076941) (width 0.75) (layer F.Cu) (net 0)))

